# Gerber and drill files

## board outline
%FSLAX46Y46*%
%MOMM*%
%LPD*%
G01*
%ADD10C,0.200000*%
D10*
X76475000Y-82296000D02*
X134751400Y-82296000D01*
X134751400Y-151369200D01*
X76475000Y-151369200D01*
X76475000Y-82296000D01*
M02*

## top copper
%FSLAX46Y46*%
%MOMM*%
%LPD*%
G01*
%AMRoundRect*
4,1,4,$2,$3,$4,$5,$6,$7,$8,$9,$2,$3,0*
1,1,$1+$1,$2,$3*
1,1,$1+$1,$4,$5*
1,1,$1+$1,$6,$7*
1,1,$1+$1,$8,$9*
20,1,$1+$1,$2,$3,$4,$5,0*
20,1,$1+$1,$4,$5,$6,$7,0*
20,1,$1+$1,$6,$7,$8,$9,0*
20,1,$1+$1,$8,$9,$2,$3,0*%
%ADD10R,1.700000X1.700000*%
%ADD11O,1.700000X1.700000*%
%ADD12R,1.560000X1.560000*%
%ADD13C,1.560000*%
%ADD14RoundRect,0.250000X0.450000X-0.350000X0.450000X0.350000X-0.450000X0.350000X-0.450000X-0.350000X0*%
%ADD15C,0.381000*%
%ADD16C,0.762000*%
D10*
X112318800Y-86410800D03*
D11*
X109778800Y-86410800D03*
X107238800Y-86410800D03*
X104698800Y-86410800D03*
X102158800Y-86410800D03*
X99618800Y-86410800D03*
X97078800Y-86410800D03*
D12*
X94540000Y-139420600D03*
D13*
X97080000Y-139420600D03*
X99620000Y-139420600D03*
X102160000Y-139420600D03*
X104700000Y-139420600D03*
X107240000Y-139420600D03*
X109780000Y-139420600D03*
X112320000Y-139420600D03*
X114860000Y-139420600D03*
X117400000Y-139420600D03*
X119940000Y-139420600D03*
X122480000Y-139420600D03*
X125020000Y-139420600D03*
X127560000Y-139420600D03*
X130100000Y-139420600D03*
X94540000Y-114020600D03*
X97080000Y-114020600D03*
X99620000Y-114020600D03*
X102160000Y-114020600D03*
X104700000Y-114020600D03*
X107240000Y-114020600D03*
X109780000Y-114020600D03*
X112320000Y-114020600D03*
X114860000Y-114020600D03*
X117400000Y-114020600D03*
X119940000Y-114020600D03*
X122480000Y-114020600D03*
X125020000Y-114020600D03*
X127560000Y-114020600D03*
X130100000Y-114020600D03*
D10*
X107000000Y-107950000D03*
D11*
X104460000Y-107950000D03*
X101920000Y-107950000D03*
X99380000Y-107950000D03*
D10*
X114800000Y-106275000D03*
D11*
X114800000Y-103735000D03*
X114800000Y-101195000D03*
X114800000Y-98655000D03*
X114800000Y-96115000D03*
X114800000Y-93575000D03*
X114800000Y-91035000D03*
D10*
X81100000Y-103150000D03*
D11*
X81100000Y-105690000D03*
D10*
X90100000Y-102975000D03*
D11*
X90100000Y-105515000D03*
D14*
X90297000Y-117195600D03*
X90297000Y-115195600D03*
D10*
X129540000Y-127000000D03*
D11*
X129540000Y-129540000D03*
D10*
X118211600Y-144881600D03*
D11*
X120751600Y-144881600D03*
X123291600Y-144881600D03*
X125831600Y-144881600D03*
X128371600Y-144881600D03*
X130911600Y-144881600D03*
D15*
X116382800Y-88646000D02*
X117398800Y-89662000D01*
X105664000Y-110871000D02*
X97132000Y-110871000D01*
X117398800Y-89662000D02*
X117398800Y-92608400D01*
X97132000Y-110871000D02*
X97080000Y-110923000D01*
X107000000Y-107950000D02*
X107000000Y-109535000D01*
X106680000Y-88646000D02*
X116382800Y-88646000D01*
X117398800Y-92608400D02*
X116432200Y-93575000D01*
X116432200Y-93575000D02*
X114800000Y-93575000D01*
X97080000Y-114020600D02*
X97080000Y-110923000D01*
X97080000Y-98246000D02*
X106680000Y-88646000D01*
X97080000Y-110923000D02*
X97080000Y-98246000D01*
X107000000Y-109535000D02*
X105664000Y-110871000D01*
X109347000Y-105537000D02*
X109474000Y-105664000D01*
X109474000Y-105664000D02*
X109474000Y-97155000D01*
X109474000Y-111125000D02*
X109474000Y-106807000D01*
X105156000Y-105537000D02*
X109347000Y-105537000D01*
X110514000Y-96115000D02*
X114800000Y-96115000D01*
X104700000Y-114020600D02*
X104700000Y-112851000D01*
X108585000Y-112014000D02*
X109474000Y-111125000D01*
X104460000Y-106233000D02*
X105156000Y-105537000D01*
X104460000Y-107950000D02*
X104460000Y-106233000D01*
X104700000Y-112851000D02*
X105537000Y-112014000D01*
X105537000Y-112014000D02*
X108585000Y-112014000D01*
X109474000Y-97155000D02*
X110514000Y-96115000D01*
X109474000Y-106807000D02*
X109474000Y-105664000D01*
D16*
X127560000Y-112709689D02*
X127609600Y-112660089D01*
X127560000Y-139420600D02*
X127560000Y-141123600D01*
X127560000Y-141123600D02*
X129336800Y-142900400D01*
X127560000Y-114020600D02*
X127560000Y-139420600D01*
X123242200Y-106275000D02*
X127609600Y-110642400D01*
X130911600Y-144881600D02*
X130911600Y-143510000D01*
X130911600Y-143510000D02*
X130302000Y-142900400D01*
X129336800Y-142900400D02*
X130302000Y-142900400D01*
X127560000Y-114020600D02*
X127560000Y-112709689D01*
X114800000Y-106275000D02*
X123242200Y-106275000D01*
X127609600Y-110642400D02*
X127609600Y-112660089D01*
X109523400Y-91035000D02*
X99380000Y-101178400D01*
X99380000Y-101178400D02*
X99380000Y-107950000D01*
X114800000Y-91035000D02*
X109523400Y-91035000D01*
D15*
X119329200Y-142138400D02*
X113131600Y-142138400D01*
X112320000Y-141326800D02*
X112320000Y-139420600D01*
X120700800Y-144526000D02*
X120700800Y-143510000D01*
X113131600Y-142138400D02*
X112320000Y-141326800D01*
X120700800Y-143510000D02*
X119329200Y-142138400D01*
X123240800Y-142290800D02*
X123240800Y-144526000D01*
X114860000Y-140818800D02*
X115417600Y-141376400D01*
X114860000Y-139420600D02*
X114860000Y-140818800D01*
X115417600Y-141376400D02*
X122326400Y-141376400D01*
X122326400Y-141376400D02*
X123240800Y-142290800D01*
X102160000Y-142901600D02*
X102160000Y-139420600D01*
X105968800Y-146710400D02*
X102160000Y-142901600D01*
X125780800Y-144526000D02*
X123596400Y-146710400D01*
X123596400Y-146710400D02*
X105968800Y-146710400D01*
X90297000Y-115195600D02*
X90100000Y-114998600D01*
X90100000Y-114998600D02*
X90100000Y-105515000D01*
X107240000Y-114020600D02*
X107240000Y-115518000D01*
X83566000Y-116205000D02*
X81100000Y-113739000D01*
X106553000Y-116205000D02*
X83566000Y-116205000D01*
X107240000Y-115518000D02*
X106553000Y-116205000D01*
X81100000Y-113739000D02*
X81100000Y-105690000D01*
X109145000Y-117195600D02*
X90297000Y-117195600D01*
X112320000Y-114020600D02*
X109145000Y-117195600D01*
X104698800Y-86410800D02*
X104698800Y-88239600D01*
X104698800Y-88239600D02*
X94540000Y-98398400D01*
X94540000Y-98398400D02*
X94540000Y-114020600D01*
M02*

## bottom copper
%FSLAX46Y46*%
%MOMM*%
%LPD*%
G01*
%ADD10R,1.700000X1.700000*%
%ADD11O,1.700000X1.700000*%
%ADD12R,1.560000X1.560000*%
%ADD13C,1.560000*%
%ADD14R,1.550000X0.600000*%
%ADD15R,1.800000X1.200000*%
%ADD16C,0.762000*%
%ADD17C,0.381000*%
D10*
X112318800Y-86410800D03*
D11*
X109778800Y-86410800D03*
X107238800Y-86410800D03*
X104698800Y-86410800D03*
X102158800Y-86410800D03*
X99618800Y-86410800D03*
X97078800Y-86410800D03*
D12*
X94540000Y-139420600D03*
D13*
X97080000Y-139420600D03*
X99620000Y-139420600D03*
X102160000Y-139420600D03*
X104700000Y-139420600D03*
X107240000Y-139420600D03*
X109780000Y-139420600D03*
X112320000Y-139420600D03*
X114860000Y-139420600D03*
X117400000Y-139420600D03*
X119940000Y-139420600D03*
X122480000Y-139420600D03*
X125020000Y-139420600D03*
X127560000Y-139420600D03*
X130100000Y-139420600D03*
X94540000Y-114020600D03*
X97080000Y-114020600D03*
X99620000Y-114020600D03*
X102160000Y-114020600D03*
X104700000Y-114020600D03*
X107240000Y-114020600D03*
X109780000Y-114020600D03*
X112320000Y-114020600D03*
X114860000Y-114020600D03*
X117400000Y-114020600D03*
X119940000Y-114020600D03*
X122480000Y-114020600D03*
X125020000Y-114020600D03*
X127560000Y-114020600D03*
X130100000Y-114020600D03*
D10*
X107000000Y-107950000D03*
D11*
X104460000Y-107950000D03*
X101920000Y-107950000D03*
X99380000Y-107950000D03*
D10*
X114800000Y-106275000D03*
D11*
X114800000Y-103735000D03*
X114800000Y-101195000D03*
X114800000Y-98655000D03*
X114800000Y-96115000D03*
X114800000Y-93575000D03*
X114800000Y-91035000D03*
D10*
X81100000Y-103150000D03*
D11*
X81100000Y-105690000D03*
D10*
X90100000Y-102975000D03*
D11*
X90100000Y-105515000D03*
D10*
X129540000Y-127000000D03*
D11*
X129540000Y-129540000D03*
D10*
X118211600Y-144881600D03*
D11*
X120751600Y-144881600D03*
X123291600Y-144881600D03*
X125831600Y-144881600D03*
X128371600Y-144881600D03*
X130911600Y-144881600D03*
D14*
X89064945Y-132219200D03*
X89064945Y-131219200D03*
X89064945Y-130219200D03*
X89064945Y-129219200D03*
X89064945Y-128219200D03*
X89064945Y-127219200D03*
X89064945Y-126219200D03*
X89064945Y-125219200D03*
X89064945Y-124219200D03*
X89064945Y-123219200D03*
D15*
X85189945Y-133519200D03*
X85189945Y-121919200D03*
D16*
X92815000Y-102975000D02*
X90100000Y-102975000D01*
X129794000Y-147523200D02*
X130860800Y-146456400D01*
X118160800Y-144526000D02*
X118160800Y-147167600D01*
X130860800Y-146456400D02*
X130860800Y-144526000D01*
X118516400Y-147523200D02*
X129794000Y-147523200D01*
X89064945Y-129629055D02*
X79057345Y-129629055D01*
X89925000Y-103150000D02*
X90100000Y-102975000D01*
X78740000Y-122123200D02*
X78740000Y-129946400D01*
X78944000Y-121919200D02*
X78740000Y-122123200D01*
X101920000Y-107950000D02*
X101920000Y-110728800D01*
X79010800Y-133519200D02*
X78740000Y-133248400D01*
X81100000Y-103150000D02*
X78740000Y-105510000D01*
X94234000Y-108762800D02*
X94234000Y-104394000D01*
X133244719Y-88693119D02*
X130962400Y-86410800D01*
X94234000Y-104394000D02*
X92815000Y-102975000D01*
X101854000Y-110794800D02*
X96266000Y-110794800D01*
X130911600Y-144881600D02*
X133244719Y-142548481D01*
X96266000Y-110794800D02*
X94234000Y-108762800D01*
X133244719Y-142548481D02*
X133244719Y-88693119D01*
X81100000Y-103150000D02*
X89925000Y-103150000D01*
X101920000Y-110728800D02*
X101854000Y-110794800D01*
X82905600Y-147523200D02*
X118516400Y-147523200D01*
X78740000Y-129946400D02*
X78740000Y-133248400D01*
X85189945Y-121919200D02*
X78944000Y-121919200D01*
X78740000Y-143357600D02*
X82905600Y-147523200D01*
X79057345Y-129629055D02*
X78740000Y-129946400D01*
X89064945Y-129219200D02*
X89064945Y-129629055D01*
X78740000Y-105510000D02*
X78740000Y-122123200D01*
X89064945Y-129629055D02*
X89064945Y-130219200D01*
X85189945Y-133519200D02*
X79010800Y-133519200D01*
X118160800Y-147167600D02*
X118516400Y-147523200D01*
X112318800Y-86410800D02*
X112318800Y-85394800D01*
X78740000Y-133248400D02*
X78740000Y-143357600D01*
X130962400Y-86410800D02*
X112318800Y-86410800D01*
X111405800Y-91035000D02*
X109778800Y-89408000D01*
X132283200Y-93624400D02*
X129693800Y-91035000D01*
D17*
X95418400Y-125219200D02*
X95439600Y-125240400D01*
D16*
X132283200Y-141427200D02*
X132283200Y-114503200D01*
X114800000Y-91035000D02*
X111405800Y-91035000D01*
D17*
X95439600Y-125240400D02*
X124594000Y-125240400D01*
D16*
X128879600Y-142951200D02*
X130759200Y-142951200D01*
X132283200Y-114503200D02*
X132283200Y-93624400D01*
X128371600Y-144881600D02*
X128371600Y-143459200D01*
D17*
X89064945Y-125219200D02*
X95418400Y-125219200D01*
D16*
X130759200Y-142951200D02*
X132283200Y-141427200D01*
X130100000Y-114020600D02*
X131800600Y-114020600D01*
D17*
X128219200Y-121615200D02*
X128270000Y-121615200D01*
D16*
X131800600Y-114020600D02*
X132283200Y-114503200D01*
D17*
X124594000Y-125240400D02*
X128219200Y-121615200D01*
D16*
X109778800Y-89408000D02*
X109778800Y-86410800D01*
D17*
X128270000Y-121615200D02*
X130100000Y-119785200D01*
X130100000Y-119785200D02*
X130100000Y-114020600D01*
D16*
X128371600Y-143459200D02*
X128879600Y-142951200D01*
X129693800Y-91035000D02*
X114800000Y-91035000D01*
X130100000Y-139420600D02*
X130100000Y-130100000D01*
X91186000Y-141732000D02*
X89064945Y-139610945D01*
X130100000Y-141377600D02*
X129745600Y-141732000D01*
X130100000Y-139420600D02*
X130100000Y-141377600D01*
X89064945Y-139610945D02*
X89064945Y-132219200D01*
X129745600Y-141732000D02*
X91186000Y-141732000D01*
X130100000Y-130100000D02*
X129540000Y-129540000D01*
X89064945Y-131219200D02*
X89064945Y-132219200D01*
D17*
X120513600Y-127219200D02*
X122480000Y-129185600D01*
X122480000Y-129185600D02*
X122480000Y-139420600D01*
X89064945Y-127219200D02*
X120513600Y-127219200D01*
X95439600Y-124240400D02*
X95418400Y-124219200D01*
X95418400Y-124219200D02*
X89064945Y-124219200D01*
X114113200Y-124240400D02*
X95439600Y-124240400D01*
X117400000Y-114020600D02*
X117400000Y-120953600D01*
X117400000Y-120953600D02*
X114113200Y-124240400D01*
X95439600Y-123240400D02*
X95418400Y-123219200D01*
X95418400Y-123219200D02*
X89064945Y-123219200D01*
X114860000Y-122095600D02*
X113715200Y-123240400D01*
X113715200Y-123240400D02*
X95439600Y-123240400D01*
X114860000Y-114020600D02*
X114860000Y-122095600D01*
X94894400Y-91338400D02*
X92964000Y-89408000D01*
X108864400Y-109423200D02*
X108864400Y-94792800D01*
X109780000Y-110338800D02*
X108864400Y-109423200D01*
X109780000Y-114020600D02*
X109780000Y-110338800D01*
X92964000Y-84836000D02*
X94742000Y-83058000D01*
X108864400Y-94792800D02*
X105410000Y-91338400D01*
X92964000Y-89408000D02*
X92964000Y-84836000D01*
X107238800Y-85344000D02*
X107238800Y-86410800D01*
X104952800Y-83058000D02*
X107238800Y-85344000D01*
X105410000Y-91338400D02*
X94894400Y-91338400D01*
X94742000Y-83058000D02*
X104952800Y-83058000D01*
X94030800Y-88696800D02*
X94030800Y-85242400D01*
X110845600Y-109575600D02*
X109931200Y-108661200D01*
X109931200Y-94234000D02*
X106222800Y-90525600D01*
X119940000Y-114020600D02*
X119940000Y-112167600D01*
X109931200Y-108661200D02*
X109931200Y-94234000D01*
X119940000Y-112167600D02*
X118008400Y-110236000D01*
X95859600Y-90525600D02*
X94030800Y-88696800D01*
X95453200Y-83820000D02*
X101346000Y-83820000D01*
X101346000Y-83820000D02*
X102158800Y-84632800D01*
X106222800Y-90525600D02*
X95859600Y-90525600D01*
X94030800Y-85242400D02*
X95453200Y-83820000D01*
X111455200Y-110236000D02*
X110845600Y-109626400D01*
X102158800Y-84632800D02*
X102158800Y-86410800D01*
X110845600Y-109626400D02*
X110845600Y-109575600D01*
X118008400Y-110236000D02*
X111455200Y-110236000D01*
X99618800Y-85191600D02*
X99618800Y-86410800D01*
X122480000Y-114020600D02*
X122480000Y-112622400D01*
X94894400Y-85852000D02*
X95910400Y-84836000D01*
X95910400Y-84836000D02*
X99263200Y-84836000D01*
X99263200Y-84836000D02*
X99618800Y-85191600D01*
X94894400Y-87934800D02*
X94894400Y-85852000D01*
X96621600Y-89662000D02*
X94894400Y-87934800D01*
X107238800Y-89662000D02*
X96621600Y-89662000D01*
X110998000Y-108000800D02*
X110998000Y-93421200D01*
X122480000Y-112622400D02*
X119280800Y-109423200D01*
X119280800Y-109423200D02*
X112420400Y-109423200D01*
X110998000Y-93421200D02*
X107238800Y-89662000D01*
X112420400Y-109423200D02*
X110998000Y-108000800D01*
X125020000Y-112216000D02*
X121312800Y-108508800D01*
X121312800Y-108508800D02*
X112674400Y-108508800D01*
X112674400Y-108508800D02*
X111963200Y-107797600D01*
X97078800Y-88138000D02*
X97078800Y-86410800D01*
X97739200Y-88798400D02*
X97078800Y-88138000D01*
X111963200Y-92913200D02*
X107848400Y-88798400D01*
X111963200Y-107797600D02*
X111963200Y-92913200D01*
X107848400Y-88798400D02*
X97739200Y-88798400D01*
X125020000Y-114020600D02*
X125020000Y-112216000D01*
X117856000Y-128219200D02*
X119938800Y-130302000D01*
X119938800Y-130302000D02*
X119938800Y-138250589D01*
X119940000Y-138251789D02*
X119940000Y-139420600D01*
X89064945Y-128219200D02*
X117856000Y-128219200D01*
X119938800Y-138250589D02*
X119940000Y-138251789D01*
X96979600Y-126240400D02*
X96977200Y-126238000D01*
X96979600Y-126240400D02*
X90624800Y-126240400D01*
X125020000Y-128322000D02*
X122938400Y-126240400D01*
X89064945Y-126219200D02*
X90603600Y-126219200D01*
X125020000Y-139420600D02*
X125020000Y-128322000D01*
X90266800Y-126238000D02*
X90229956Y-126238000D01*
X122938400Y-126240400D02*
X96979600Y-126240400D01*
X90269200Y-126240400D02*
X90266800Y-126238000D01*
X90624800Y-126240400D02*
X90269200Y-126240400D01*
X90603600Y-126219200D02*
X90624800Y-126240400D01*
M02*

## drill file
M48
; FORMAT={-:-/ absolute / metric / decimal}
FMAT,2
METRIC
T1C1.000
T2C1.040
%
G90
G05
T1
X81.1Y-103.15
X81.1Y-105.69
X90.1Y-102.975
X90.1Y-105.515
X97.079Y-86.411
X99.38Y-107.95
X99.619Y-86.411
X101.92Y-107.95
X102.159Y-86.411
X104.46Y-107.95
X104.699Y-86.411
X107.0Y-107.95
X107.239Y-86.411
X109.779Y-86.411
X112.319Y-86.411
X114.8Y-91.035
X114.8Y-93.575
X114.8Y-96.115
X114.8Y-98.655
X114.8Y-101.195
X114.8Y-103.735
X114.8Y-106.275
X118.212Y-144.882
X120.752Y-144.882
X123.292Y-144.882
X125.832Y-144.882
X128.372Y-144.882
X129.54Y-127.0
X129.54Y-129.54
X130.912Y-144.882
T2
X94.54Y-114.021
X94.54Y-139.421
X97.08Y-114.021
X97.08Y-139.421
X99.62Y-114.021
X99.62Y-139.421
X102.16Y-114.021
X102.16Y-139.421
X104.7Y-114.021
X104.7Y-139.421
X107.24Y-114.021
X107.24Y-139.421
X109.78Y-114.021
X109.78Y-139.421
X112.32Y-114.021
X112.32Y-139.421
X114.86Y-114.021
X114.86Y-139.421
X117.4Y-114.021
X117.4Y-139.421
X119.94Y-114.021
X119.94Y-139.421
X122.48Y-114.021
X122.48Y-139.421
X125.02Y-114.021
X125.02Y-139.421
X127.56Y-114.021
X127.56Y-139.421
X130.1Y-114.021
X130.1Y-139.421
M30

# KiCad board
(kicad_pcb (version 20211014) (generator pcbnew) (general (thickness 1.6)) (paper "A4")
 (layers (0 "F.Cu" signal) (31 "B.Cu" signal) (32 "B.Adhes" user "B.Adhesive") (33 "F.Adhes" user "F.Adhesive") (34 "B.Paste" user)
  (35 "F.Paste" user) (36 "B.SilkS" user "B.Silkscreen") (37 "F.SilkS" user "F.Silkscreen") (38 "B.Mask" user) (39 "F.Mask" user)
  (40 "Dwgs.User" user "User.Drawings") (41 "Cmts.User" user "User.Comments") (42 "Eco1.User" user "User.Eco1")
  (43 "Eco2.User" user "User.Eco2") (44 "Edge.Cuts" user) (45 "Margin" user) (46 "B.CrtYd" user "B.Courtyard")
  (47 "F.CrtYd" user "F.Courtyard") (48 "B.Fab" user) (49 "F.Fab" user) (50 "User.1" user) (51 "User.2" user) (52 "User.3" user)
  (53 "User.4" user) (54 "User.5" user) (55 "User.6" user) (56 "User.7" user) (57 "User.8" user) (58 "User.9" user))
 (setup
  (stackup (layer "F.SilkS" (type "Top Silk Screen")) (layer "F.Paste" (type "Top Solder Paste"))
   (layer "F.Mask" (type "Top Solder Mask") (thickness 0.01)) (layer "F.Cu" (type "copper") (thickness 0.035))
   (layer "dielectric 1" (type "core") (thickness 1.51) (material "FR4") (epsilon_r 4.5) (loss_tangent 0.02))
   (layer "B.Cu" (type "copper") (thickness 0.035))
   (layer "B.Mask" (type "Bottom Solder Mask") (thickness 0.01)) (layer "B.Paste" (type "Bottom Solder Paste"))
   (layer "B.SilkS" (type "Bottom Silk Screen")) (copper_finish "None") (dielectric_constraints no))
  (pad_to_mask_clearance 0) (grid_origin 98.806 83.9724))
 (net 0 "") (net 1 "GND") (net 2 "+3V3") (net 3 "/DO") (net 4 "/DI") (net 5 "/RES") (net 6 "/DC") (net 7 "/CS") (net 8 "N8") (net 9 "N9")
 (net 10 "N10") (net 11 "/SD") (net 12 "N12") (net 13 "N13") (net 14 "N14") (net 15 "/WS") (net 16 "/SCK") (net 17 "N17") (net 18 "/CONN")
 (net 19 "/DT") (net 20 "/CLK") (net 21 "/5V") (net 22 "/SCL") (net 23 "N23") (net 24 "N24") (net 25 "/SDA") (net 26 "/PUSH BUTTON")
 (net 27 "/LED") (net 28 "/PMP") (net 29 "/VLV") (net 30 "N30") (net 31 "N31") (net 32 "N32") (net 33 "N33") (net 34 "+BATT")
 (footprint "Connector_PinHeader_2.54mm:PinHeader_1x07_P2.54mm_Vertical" (layer "F.Cu") (at 112.3188 86.4108 -90)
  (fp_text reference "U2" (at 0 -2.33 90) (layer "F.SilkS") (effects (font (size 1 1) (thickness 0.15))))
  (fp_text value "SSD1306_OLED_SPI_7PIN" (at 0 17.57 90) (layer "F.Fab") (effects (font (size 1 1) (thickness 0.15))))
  (pad "1" thru_hole rect (at 0 0 270) (size 1.7 1.7) (drill 1) (layers *.Cu *.Mask) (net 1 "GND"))
  (pad "2" thru_hole oval (at 0 2.54 270) (size 1.7 1.7) (drill 1) (layers *.Cu *.Mask) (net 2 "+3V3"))
  (pad "3" thru_hole oval (at 0 5.08 270) (size 1.7 1.7) (drill 1) (layers *.Cu *.Mask) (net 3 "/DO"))
  (pad "4" thru_hole oval (at 0 7.62 270) (size 1.7 1.7) (drill 1) (layers *.Cu *.Mask) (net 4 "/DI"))
  (pad "5" thru_hole oval (at 0 10.16 270) (size 1.7 1.7) (drill 1) (layers *.Cu *.Mask) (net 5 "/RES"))
  (pad "6" thru_hole oval (at 0 12.7 270) (size 1.7 1.7) (drill 1) (layers *.Cu *.Mask) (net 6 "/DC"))
  (pad "7" thru_hole oval (at 0 15.24 270) (size 1.7 1.7) (drill 1) (layers *.Cu *.Mask) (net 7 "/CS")))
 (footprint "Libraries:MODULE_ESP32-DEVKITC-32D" (layer "F.Cu") (at 114.3 126.7206 90)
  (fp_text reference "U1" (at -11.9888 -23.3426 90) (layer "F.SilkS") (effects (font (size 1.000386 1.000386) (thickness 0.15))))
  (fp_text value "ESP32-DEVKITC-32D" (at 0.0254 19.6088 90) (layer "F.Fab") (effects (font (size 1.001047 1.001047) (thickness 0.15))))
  (pad "1" thru_hole rect (at -12.7 -19.76 90) (size 1.56 1.56) (drill 1.04) (layers *.Cu *.Mask) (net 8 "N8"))
  (pad "2" thru_hole circle (at -12.7 -17.22 90) (size 1.56 1.56) (drill 1.04) (layers *.Cu *.Mask) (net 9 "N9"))
  (pad "3" thru_hole circle (at -12.7 -14.68 90) (size 1.56 1.56) (drill 1.04) (layers *.Cu *.Mask) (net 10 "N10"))
  (pad "4" thru_hole circle (at -12.7 -12.14 90) (size 1.56 1.56) (drill 1.04) (layers *.Cu *.Mask) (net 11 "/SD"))
  (pad "5" thru_hole circle (at -12.7 -9.6 90) (size 1.56 1.56) (drill 1.04) (layers *.Cu *.Mask) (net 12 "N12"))
  (pad "6" thru_hole circle (at -12.7 -7.06 90) (size 1.56 1.56) (drill 1.04) (layers *.Cu *.Mask) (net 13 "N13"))
  (pad "7" thru_hole circle (at -12.7 -4.52 90) (size 1.56 1.56) (drill 1.04) (layers *.Cu *.Mask) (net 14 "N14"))
  (pad "8" thru_hole circle (at -12.7 -1.98 90) (size 1.56 1.56) (drill 1.04) (layers *.Cu *.Mask) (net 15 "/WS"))
  (pad "9" thru_hole circle (at -12.7 0.56 90) (size 1.56 1.56) (drill 1.04) (layers *.Cu *.Mask) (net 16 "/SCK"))
  (pad "10" thru_hole circle (at -12.7 3.1 90) (size 1.56 1.56) (drill 1.04) (layers *.Cu *.Mask) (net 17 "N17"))
  (pad "11" thru_hole circle (at -12.7 5.64 90) (size 1.56 1.56) (drill 1.04) (layers *.Cu *.Mask) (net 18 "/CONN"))
  (pad "12" thru_hole circle (at -12.7 8.18 90) (size 1.56 1.56) (drill 1.04) (layers *.Cu *.Mask) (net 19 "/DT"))
  (pad "13" thru_hole circle (at -12.7 10.72 90) (size 1.56 1.56) (drill 1.04) (layers *.Cu *.Mask) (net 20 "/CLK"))
  (pad "14" thru_hole circle (at -12.7 13.26 90) (size 1.56 1.56) (drill 1.04) (layers *.Cu *.Mask) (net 1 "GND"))
  (pad "15" thru_hole circle (at -12.7 15.8 90) (size 1.56 1.56) (drill 1.04) (layers *.Cu *.Mask) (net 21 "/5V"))
  (pad "16" thru_hole circle (at 12.7 -19.76 90) (size 1.56 1.56) (drill 1.04) (layers *.Cu *.Mask) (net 4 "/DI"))
  (pad "17" thru_hole circle (at 12.7 -17.22 90) (size 1.56 1.56) (drill 1.04) (layers *.Cu *.Mask) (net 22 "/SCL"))
  (pad "18" thru_hole circle (at 12.7 -14.68 90) (size 1.56 1.56) (drill 1.04) (layers *.Cu *.Mask) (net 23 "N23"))
  (pad "19" thru_hole circle (at 12.7 -12.14 90) (size 1.56 1.56) (drill 1.04) (layers *.Cu *.Mask) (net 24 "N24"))
  (pad "20" thru_hole circle (at 12.7 -9.6 90) (size 1.56 1.56) (drill 1.04) (layers *.Cu *.Mask) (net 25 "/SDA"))
  (pad "21" thru_hole circle (at 12.7 -7.06 90) (size 1.56 1.56) (drill 1.04) (layers *.Cu *.Mask) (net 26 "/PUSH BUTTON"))
  (pad "22" thru_hole circle (at 12.7 -4.52 90) (size 1.56 1.56) (drill 1.04) (layers *.Cu *.Mask) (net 3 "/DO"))
  (pad "23" thru_hole circle (at 12.7 -1.98 90) (size 1.56 1.56) (drill 1.04) (layers *.Cu *.Mask) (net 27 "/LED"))
  (pad "24" thru_hole circle (at 12.7 0.56 90) (size 1.56 1.56) (drill 1.04) (layers *.Cu *.Mask) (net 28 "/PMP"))
  (pad "25" thru_hole circle (at 12.7 3.1 90) (size 1.56 1.56) (drill 1.04) (layers *.Cu *.Mask) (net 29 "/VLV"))
  (pad "26" thru_hole circle (at 12.7 5.64 90) (size 1.56 1.56) (drill 1.04) (layers *.Cu *.Mask) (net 5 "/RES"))
  (pad "27" thru_hole circle (at 12.7 8.18 90) (size 1.56 1.56) (drill 1.04) (layers *.Cu *.Mask) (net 6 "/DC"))
  (pad "28" thru_hole circle (at 12.7 10.72 90) (size 1.56 1.56) (drill 1.04) (layers *.Cu *.Mask) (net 7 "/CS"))
  (pad "29" thru_hole circle (at 12.7 13.26 90) (size 1.56 1.56) (drill 1.04) (layers *.Cu *.Mask) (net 1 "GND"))
  (pad "30" thru_hole circle (at 12.7 15.8 90) (size 1.56 1.56) (drill 1.04) (layers *.Cu *.Mask) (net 2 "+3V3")))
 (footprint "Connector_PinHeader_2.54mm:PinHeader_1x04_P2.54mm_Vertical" (layer "F.Cu") (at 107 107.95 -90)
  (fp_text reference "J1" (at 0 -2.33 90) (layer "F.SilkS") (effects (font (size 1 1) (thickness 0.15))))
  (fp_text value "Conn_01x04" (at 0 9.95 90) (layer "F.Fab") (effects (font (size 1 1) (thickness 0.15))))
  (pad "1" thru_hole rect (at 0 0 270) (size 1.7 1.7) (drill 1) (layers *.Cu *.Mask) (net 22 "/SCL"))
  (pad "2" thru_hole oval (at 0 2.54 270) (size 1.7 1.7) (drill 1) (layers *.Cu *.Mask) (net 25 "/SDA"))
  (pad "3" thru_hole oval (at 0 5.08 270) (size 1.7 1.7) (drill 1) (layers *.Cu *.Mask) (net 1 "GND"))
  (pad "4" thru_hole oval (at 0 7.62 270) (size 1.7 1.7) (drill 1) (layers *.Cu *.Mask) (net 2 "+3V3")))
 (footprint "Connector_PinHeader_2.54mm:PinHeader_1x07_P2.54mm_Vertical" (layer "F.Cu") (at 114.8 106.275 180)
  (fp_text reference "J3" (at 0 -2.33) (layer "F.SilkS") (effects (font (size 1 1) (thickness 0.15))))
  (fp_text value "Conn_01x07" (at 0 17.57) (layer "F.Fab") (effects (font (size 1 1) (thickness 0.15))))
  (pad "1" thru_hole rect (at 0 0 180) (size 1.7 1.7) (drill 1) (layers *.Cu *.Mask) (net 1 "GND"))
  (pad "2" thru_hole oval (at 0 2.54 180) (size 1.7 1.7) (drill 1) (layers *.Cu *.Mask) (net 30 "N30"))
  (pad "3" thru_hole oval (at 0 5.08 180) (size 1.7 1.7) (drill 1) (layers *.Cu *.Mask) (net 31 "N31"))
  (pad "4" thru_hole oval (at 0 7.62 180) (size 1.7 1.7) (drill 1) (layers *.Cu *.Mask) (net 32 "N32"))
  (pad "5" thru_hole oval (at 0 10.16 180) (size 1.7 1.7) (drill 1) (layers *.Cu *.Mask) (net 25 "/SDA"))
  (pad "6" thru_hole oval (at 0 12.7 180) (size 1.7 1.7) (drill 1) (layers *.Cu *.Mask) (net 22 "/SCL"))
  (pad "7" thru_hole oval (at 0 15.24 180) (size 1.7 1.7) (drill 1) (layers *.Cu *.Mask) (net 2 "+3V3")))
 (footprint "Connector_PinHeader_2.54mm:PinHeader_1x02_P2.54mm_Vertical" (layer "F.Cu") (at 81.1 103.15)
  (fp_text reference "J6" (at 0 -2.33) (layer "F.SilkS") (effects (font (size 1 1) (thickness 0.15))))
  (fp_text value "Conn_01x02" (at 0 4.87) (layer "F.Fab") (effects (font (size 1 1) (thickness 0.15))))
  (pad "1" thru_hole rect (at 0 0) (size 1.7 1.7) (drill 1) (layers *.Cu *.Mask) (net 1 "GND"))
  (pad "2" thru_hole oval (at 0 2.54) (size 1.7 1.7) (drill 1) (layers *.Cu *.Mask) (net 26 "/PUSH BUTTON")))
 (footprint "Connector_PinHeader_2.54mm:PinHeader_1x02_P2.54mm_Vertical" (layer "F.Cu") (at 90.1 102.975)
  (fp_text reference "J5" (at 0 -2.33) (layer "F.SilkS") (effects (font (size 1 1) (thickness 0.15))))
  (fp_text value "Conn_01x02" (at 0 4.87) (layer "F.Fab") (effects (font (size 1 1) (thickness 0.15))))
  (pad "1" thru_hole rect (at 0 0) (size 1.7 1.7) (drill 1) (layers *.Cu *.Mask) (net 1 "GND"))
  (pad "2" thru_hole oval (at 0 2.54) (size 1.7 1.7) (drill 1) (layers *.Cu *.Mask) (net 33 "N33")))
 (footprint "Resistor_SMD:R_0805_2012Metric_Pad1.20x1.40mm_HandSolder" (layer "F.Cu") (at 90.297 116.1956 90)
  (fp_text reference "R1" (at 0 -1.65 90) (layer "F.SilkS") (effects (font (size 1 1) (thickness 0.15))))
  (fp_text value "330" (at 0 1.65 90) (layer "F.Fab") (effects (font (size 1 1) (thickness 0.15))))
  (pad "1" smd roundrect (at -1 0 90) (size 1.2 1.4) (layers "F.Cu" "F.Paste" "F.Mask") (roundrect_rratio 0.208333) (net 27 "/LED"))
  (pad "2" smd roundrect (at 1 0 90) (size 1.2 1.4) (layers "F.Cu" "F.Paste" "F.Mask") (roundrect_rratio 0.208333) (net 33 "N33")))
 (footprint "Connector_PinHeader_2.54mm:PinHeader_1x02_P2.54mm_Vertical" (layer "F.Cu") (at 129.54 127)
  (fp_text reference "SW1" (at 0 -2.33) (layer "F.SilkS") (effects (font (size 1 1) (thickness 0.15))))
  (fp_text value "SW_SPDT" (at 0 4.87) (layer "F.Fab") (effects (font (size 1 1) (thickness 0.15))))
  (pad "1" thru_hole rect (at 0 0) (size 1.7 1.7) (drill 1) (layers *.Cu *.Mask) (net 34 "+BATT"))
  (pad "3" thru_hole oval (at 0 2.54) (size 1.7 1.7) (drill 1) (layers *.Cu *.Mask) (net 21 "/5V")))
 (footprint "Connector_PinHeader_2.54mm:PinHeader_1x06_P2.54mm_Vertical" (layer "B.Cu") (at 118.2116 144.8816 -90)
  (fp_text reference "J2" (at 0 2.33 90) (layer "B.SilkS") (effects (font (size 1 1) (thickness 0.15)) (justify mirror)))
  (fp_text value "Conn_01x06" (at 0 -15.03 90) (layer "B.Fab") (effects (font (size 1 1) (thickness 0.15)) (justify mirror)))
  (pad "1" thru_hole rect (at 0 0 270) (size 1.7 1.7) (drill 1) (layers *.Cu *.Mask) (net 1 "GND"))
  (pad "2" thru_hole oval (at 0 -2.54 270) (size 1.7 1.7) (drill 1) (layers *.Cu *.Mask) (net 15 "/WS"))
  (pad "3" thru_hole oval (at 0 -5.08 270) (size 1.7 1.7) (drill 1) (layers *.Cu *.Mask) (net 16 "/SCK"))
  (pad "4" thru_hole oval (at 0 -7.62 270) (size 1.7 1.7) (drill 1) (layers *.Cu *.Mask) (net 11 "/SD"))
  (pad "5" thru_hole oval (at 0 -10.16 270) (size 1.7 1.7) (drill 1) (layers *.Cu *.Mask) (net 2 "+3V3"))
  (pad "6" thru_hole oval (at 0 -12.7 270) (size 1.7 1.7) (drill 1) (layers *.Cu *.Mask) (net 1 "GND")))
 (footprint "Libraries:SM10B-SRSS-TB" (layer "B.Cu") (at 88.722945 133.7192 90)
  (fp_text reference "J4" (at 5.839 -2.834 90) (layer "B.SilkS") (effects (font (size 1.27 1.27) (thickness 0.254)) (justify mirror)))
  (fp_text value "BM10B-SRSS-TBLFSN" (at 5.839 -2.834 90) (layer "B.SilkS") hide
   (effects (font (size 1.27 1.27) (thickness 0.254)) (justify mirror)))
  (pad "1" smd rect locked (at 1.5 0.342 90) (size 0.6 1.55) (layers "B.Cu" "B.Paste" "B.Mask") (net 21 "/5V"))
  (pad "2" smd rect locked (at 2.5 0.342 90) (size 0.6 1.55) (layers "B.Cu" "B.Paste" "B.Mask") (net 21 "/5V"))
  (pad "3" smd rect locked (at 3.5 0.342 90) (size 0.6 1.55) (layers "B.Cu" "B.Paste" "B.Mask") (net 1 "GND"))
  (pad "4" smd rect locked (at 4.5 0.342 90) (size 0.6 1.55) (layers "B.Cu" "B.Paste" "B.Mask") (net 1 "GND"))
  (pad "5" smd rect locked (at 5.5 0.342 90) (size 0.6 1.55) (layers "B.Cu" "B.Paste" "B.Mask") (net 18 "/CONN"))
  (pad "6" smd rect locked (at 6.5 0.342 90) (size 0.6 1.55) (layers "B.Cu" "B.Paste" "B.Mask") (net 19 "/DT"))
  (pad "7" smd rect locked (at 7.5 0.342 90) (size 0.6 1.55) (layers "B.Cu" "B.Paste" "B.Mask") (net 20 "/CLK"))
  (pad "8" smd rect locked (at 8.5 0.342 90) (size 0.6 1.55) (layers "B.Cu" "B.Paste" "B.Mask") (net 2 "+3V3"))
  (pad "9" smd rect locked (at 9.5 0.342 90) (size 0.6 1.55) (layers "B.Cu" "B.Paste" "B.Mask") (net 29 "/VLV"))
  (pad "10" smd rect locked (at 10.5 0.342 90) (size 0.6 1.55) (layers "B.Cu" "B.Paste" "B.Mask") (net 28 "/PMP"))
  (pad "11" smd rect locked (at 0.2 -3.533 90) (size 1.2 1.8) (layers "B.Cu" "B.Paste" "B.Mask"))
  (pad "12" smd rect locked (at 11.8 -3.533 90) (size 1.2 1.8) (layers "B.Cu" "B.Paste" "B.Mask")))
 (gr_rect (start 76.475 82.296) (end 134.7514 151.3692) (layer "Edge.Cuts") (width 0.2) (fill none))
 (segment (start 116.3828 88.646) (end 117.3988 89.662) (width 0.381) (layer "F.Cu") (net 22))
 (segment (start 105.664 110.871) (end 97.132 110.871) (width 0.381) (layer "F.Cu") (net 22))
 (segment (start 117.3988 89.662) (end 117.3988 92.6084) (width 0.381) (layer "F.Cu") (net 22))
 (segment (start 97.132 110.871) (end 97.08 110.923) (width 0.381) (layer "F.Cu") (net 22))
 (segment (start 107 107.95) (end 107 109.535) (width 0.381) (layer "F.Cu") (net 22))
 (segment (start 106.68 88.646) (end 116.3828 88.646) (width 0.381) (layer "F.Cu") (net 22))
 (segment (start 117.3988 92.6084) (end 116.4322 93.575) (width 0.381) (layer "F.Cu") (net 22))
 (segment (start 116.4322 93.575) (end 114.8 93.575) (width 0.381) (layer "F.Cu") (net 22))
 (segment (start 97.08 114.0206) (end 97.08 110.923) (width 0.381) (layer "F.Cu") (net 22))
 (segment (start 97.08 98.246) (end 106.68 88.646) (width 0.381) (layer "F.Cu") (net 22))
 (segment (start 97.08 110.923) (end 97.08 98.246) (width 0.381) (layer "F.Cu") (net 22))
 (segment (start 107 109.535) (end 105.664 110.871) (width 0.381) (layer "F.Cu") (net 22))
 (segment (start 109.347 105.537) (end 109.474 105.664) (width 0.381) (layer "F.Cu") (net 25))
 (segment (start 109.474 105.664) (end 109.474 97.155) (width 0.381) (layer "F.Cu") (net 25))
 (segment (start 109.474 111.125) (end 109.474 106.807) (width 0.381) (layer "F.Cu") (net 25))
 (segment (start 105.156 105.537) (end 109.347 105.537) (width 0.381) (layer "F.Cu") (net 25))
 (segment (start 110.514 96.115) (end 114.8 96.115) (width 0.381) (layer "F.Cu") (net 25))
 (segment (start 104.7 114.0206) (end 104.7 112.851) (width 0.381) (layer "F.Cu") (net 25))
 (segment (start 108.585 112.014) (end 109.474 111.125) (width 0.381) (layer "F.Cu") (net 25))
 (segment (start 104.46 106.233) (end 105.156 105.537) (width 0.381) (layer "F.Cu") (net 25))
 (segment (start 104.46 107.95) (end 104.46 106.233) (width 0.381) (layer "F.Cu") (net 25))
 (segment (start 104.7 112.851) (end 105.537 112.014) (width 0.381) (layer "F.Cu") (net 25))
 (segment (start 105.537 112.014) (end 108.585 112.014) (width 0.381) (layer "F.Cu") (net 25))
 (segment (start 109.474 97.155) (end 110.514 96.115) (width 0.381) (layer "F.Cu") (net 25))
 (segment (start 109.474 106.807) (end 109.474 105.664) (width 0.381) (layer "F.Cu") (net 25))
 (segment (start 127.56 112.709689) (end 127.6096 112.660089) (width 0.762) (layer "F.Cu") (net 1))
 (segment (start 127.56 139.4206) (end 127.56 141.1236) (width 0.762) (layer "F.Cu") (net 1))
 (segment (start 127.56 141.1236) (end 129.3368 142.9004) (width 0.762) (layer "F.Cu") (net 1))
 (segment (start 127.56 114.0206) (end 127.56 139.4206) (width 0.762) (layer "F.Cu") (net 1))
 (segment (start 123.2422 106.275) (end 127.6096 110.6424) (width 0.762) (layer "F.Cu") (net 1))
 (segment (start 130.9116 144.8816) (end 130.9116 143.51) (width 0.762) (layer "F.Cu") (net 1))
 (segment (start 130.9116 143.51) (end 130.302 142.9004) (width 0.762) (layer "F.Cu") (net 1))
 (segment (start 129.3368 142.9004) (end 130.302 142.9004) (width 0.762) (layer "F.Cu") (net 1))
 (segment (start 127.56 114.0206) (end 127.56 112.709689) (width 0.762) (layer "F.Cu") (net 1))
 (segment (start 114.8 106.275) (end 123.2422 106.275) (width 0.762) (layer "F.Cu") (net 1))
 (segment (start 127.6096 110.6424) (end 127.6096 112.660089) (width 0.762) (layer "F.Cu") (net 1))
 (segment (start 92.815 102.975) (end 90.1 102.975) (width 0.762) (layer "B.Cu") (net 1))
 (segment (start 129.794 147.5232) (end 130.8608 146.4564) (width 0.762) (layer "B.Cu") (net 1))
 (segment (start 118.1608 144.526) (end 118.1608 147.1676) (width 0.762) (layer "B.Cu") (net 1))
 (segment (start 130.8608 146.4564) (end 130.8608 144.526) (width 0.762) (layer "B.Cu") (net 1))
 (segment (start 118.5164 147.5232) (end 129.794 147.5232) (width 0.762) (layer "B.Cu") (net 1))
 (segment (start 89.064945 129.629055) (end 79.057345 129.629055) (width 0.762) (layer "B.Cu") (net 1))
 (segment (start 89.925 103.15) (end 90.1 102.975) (width 0.762) (layer "B.Cu") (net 1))
 (segment (start 78.74 122.1232) (end 78.74 129.9464) (width 0.762) (layer "B.Cu") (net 1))
 (segment (start 78.944 121.9192) (end 78.74 122.1232) (width 0.762) (layer "B.Cu") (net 1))
 (segment (start 101.92 107.95) (end 101.92 110.7288) (width 0.762) (layer "B.Cu") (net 1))
 (segment (start 79.0108 133.5192) (end 78.74 133.2484) (width 0.762) (layer "B.Cu") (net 1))
 (segment (start 81.1 103.15) (end 78.74 105.51) (width 0.762) (layer "B.Cu") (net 1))
 (segment (start 94.234 108.7628) (end 94.234 104.394) (width 0.762) (layer "B.Cu") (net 1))
 (segment (start 133.244719 88.693119) (end 130.9624 86.4108) (width 0.762) (layer "B.Cu") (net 1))
 (segment (start 94.234 104.394) (end 92.815 102.975) (width 0.762) (layer "B.Cu") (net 1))
 (segment (start 101.854 110.7948) (end 96.266 110.7948) (width 0.762) (layer "B.Cu") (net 1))
 (segment (start 130.9116 144.8816) (end 133.244719 142.548481) (width 0.762) (layer "B.Cu") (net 1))
 (segment (start 96.266 110.7948) (end 94.234 108.7628) (width 0.762) (layer "B.Cu") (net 1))
 (segment (start 133.244719 142.548481) (end 133.244719 88.693119) (width 0.762) (layer "B.Cu") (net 1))
 (segment (start 81.1 103.15) (end 89.925 103.15) (width 0.762) (layer "B.Cu") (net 1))
 (segment (start 101.92 110.7288) (end 101.854 110.7948) (width 0.762) (layer "B.Cu") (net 1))
 (segment (start 82.9056 147.5232) (end 118.5164 147.5232) (width 0.762) (layer "B.Cu") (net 1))
 (segment (start 78.74 129.9464) (end 78.74 133.2484) (width 0.762) (layer "B.Cu") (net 1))
 (segment (start 85.189945 121.9192) (end 78.944 121.9192) (width 0.762) (layer "B.Cu") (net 1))
 (segment (start 78.74 143.3576) (end 82.9056 147.5232) (width 0.762) (layer "B.Cu") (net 1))
 (segment (start 79.057345 129.629055) (end 78.74 129.9464) (width 0.762) (layer "B.Cu") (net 1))
 (segment (start 89.064945 129.2192) (end 89.064945 129.629055) (width 0.762) (layer "B.Cu") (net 1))
 (segment (start 78.74 105.51) (end 78.74 122.1232) (width 0.762) (layer "B.Cu") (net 1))
 (segment (start 89.064945 129.629055) (end 89.064945 130.2192) (width 0.762) (layer "B.Cu") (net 1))
 (segment (start 85.189945 133.5192) (end 79.0108 133.5192) (width 0.762) (layer "B.Cu") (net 1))
 (segment (start 118.1608 147.1676) (end 118.5164 147.5232) (width 0.762) (layer "B.Cu") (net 1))
 (segment (start 112.3188 86.4108) (end 112.3188 85.3948) (width 0.762) (layer "B.Cu") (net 1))
 (segment (start 78.74 133.2484) (end 78.74 143.3576) (width 0.762) (layer "B.Cu") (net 1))
 (segment (start 130.9624 86.4108) (end 112.3188 86.4108) (width 0.762) (layer "B.Cu") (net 1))
 (segment (start 109.5234 91.035) (end 99.38 101.1784) (width 0.762) (layer "F.Cu") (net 2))
 (segment (start 99.38 101.1784) (end 99.38 107.95) (width 0.762) (layer "F.Cu") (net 2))
 (segment (start 114.8 91.035) (end 109.5234 91.035) (width 0.762) (layer "F.Cu") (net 2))
 (segment (start 111.4058 91.035) (end 109.7788 89.408) (width 0.762) (layer "B.Cu") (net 2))
 (segment (start 132.2832 93.6244) (end 129.6938 91.035) (width 0.762) (layer "B.Cu") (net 2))
 (segment (start 95.4184 125.2192) (end 95.4396 125.2404) (width 0.381) (layer "B.Cu") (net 2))
 (segment (start 132.2832 141.4272) (end 132.2832 114.5032) (width 0.762) (layer "B.Cu") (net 2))
 (segment (start 114.8 91.035) (end 111.4058 91.035) (width 0.762) (layer "B.Cu") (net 2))
 (segment (start 95.4396 125.2404) (end 124.594 125.2404) (width 0.381) (layer "B.Cu") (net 2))
 (segment (start 128.8796 142.9512) (end 130.7592 142.9512) (width 0.762) (layer "B.Cu") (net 2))
 (segment (start 132.2832 114.5032) (end 132.2832 93.6244) (width 0.762) (layer "B.Cu") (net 2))
 (segment (start 128.3716 144.8816) (end 128.3716 143.4592) (width 0.762) (layer "B.Cu") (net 2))
 (segment (start 89.064945 125.2192) (end 95.4184 125.2192) (width 0.381) (layer "B.Cu") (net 2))
 (segment (start 130.7592 142.9512) (end 132.2832 141.4272) (width 0.762) (layer "B.Cu") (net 2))
 (segment (start 130.1 114.0206) (end 131.8006 114.0206) (width 0.762) (layer "B.Cu") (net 2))
 (segment (start 128.2192 121.6152) (end 128.27 121.6152) (width 0.381) (layer "B.Cu") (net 2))
 (segment (start 131.8006 114.0206) (end 132.2832 114.5032) (width 0.762) (layer "B.Cu") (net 2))
 (segment (start 124.594 125.2404) (end 128.2192 121.6152) (width 0.381) (layer "B.Cu") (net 2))
 (segment (start 109.7788 89.408) (end 109.7788 86.4108) (width 0.762) (layer "B.Cu") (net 2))
 (segment (start 128.27 121.6152) (end 130.1 119.7852) (width 0.381) (layer "B.Cu") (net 2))
 (segment (start 130.1 119.7852) (end 130.1 114.0206) (width 0.381) (layer "B.Cu") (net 2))
 (segment (start 128.3716 143.4592) (end 128.8796 142.9512) (width 0.762) (layer "B.Cu") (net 2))
 (segment (start 129.6938 91.035) (end 114.8 91.035) (width 0.762) (layer "B.Cu") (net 2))
 (segment (start 119.3292 142.1384) (end 113.1316 142.1384) (width 0.381) (layer "F.Cu") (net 15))
 (segment (start 112.32 141.3268) (end 112.32 139.4206) (width 0.381) (layer "F.Cu") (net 15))
 (segment (start 120.7008 144.526) (end 120.7008 143.51) (width 0.381) (layer "F.Cu") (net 15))
 (segment (start 113.1316 142.1384) (end 112.32 141.3268) (width 0.381) (layer "F.Cu") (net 15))
 (segment (start 120.7008 143.51) (end 119.3292 142.1384) (width 0.381) (layer "F.Cu") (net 15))
 (segment (start 123.2408 142.2908) (end 123.2408 144.526) (width 0.381) (layer "F.Cu") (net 16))
 (segment (start 114.86 140.8188) (end 115.4176 141.3764) (width 0.381) (layer "F.Cu") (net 16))
 (segment (start 114.86 139.4206) (end 114.86 140.8188) (width 0.381) (layer "F.Cu") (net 16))
 (segment (start 115.4176 141.3764) (end 122.3264 141.3764) (width 0.381) (layer "F.Cu") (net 16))
 (segment (start 122.3264 141.3764) (end 123.2408 142.2908) (width 0.381) (layer "F.Cu") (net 16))
 (segment (start 102.16 142.9016) (end 102.16 139.4206) (width 0.381) (layer "F.Cu") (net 11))
 (segment (start 105.9688 146.7104) (end 102.16 142.9016) (width 0.381) (layer "F.Cu") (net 11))
 (segment (start 125.7808 144.526) (end 123.5964 146.7104) (width 0.381) (layer "F.Cu") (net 11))
 (segment (start 123.5964 146.7104) (end 105.9688 146.7104) (width 0.381) (layer "F.Cu") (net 11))
 (segment (start 130.1 139.4206) (end 130.1 130.1) (width 0.762) (layer "B.Cu") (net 21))
 (segment (start 91.186 141.732) (end 89.064945 139.610945) (width 0.762) (layer "B.Cu") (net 21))
 (segment (start 130.1 141.3776) (end 129.7456 141.732) (width 0.762) (layer "B.Cu") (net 21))
 (segment (start 130.1 139.4206) (end 130.1 141.3776) (width 0.762) (layer "B.Cu") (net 21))
 (segment (start 89.064945 139.610945) (end 89.064945 132.2192) (width 0.762) (layer "B.Cu") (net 21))
 (segment (start 129.7456 141.732) (end 91.186 141.732) (width 0.762) (layer "B.Cu") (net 21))
 (segment (start 130.1 130.1) (end 129.54 129.54) (width 0.762) (layer "B.Cu") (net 21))
 (segment (start 89.064945 131.2192) (end 89.064945 132.2192) (width 0.762) (layer "B.Cu") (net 21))
 (segment (start 120.5136 127.2192) (end 122.48 129.1856) (width 0.381) (layer "B.Cu") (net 19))
 (segment (start 122.48 129.1856) (end 122.48 139.4206) (width 0.381) (layer "B.Cu") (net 19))
 (segment (start 89.064945 127.2192) (end 120.5136 127.2192) (width 0.381) (layer "B.Cu") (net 19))
 (segment (start 95.4396 124.2404) (end 95.4184 124.2192) (width 0.381) (layer "B.Cu") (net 29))
 (segment (start 95.4184 124.2192) (end 89.064945 124.2192) (width 0.381) (layer "B.Cu") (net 29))
 (segment (start 114.1132 124.2404) (end 95.4396 124.2404) (width 0.381) (layer "B.Cu") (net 29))
 (segment (start 117.4 114.0206) (end 117.4 120.9536) (width 0.381) (layer "B.Cu") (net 29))
 (segment (start 117.4 120.9536) (end 114.1132 124.2404) (width 0.381) (layer "B.Cu") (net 29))
 (segment (start 95.4396 123.2404) (end 95.4184 123.2192) (width 0.381) (layer "B.Cu") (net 28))
 (segment (start 95.4184 123.2192) (end 89.064945 123.2192) (width 0.381) (layer "B.Cu") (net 28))
 (segment (start 114.86 122.0956) (end 113.7152 123.2404) (width 0.381) (layer "B.Cu") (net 28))
 (segment (start 113.7152 123.2404) (end 95.4396 123.2404) (width 0.381) (layer "B.Cu") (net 28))
 (segment (start 114.86 114.0206) (end 114.86 122.0956) (width 0.381) (layer "B.Cu") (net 28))
 (segment (start 90.297 115.1956) (end 90.1 114.9986) (width 0.381) (layer "F.Cu") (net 33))
 (segment (start 90.1 114.9986) (end 90.1 105.515) (width 0.381) (layer "F.Cu") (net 33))
 (segment (start 107.24 114.0206) (end 107.24 115.518) (width 0.381) (layer "F.Cu") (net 26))
 (segment (start 83.566 116.205) (end 81.1 113.739) (width 0.381) (layer "F.Cu") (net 26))
 (segment (start 106.553 116.205) (end 83.566 116.205) (width 0.381) (layer "F.Cu") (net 26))
 (segment (start 107.24 115.518) (end 106.553 116.205) (width 0.381) (layer "F.Cu") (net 26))
 (segment (start 81.1 113.739) (end 81.1 105.69) (width 0.381) (layer "F.Cu") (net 26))
 (segment (start 109.145 117.1956) (end 90.297 117.1956) (width 0.381) (layer "F.Cu") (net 27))
 (segment (start 112.32 114.0206) (end 109.145 117.1956) (width 0.381) (layer "F.Cu") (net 27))
 (segment (start 104.6988 86.4108) (end 104.6988 88.2396) (width 0.381) (layer "F.Cu") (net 4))
 (segment (start 104.6988 88.2396) (end 94.54 98.3984) (width 0.381) (layer "F.Cu") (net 4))
 (segment (start 94.54 98.3984) (end 94.54 114.0206) (width 0.381) (layer "F.Cu") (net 4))
 (segment (start 94.8944 91.3384) (end 92.964 89.408) (width 0.381) (layer "B.Cu") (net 3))
 (segment (start 108.8644 109.4232) (end 108.8644 94.7928) (width 0.381) (layer "B.Cu") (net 3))
 (segment (start 109.78 110.3388) (end 108.8644 109.4232) (width 0.381) (layer "B.Cu") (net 3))
 (segment (start 109.78 114.0206) (end 109.78 110.3388) (width 0.381) (layer "B.Cu") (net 3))
 (segment (start 92.964 84.836) (end 94.742 83.058) (width 0.381) (layer "B.Cu") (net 3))
 (segment (start 108.8644 94.7928) (end 105.41 91.3384) (width 0.381) (layer "B.Cu") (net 3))
 (segment (start 92.964 89.408) (end 92.964 84.836) (width 0.381) (layer "B.Cu") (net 3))
 (segment (start 107.2388 85.344) (end 107.2388 86.4108) (width 0.381) (layer "B.Cu") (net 3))
 (segment (start 104.9528 83.058) (end 107.2388 85.344) (width 0.381) (layer "B.Cu") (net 3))
 (segment (start 105.41 91.3384) (end 94.8944 91.3384) (width 0.381) (layer "B.Cu") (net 3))
 (segment (start 94.742 83.058) (end 104.9528 83.058) (width 0.381) (layer "B.Cu") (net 3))
 (segment (start 94.0308 88.6968) (end 94.0308 85.2424) (width 0.381) (layer "B.Cu") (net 5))
 (segment (start 110.8456 109.5756) (end 109.9312 108.6612) (width 0.381) (layer "B.Cu") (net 5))
 (segment (start 109.9312 94.234) (end 106.2228 90.5256) (width 0.381) (layer "B.Cu") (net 5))
 (segment (start 119.94 114.0206) (end 119.94 112.1676) (width 0.381) (layer "B.Cu") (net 5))
 (segment (start 109.9312 108.6612) (end 109.9312 94.234) (width 0.381) (layer "B.Cu") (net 5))
 (segment (start 119.94 112.1676) (end 118.0084 110.236) (width 0.381) (layer "B.Cu") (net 5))
 (segment (start 95.8596 90.5256) (end 94.0308 88.6968) (width 0.381) (layer "B.Cu") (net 5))
 (segment (start 95.4532 83.82) (end 101.346 83.82) (width 0.381) (layer "B.Cu") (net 5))
 (segment (start 101.346 83.82) (end 102.1588 84.6328) (width 0.381) (layer "B.Cu") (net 5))
 (segment (start 106.2228 90.5256) (end 95.8596 90.5256) (width 0.381) (layer "B.Cu") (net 5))
 (segment (start 94.0308 85.2424) (end 95.4532 83.82) (width 0.381) (layer "B.Cu") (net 5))
 (segment (start 111.4552 110.236) (end 110.8456 109.6264) (width 0.381) (layer "B.Cu") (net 5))
 (segment (start 102.1588 84.6328) (end 102.1588 86.4108) (width 0.381) (layer "B.Cu") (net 5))
 (segment (start 110.8456 109.6264) (end 110.8456 109.5756) (width 0.381) (layer "B.Cu") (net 5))
 (segment (start 118.0084 110.236) (end 111.4552 110.236) (width 0.381) (layer "B.Cu") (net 5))
 (segment (start 99.6188 85.1916) (end 99.6188 86.4108) (width 0.381) (layer "B.Cu") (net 6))
 (segment (start 122.48 114.0206) (end 122.48 112.6224) (width 0.381) (layer "B.Cu") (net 6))
 (segment (start 94.8944 85.852) (end 95.9104 84.836) (width 0.381) (layer "B.Cu") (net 6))
 (segment (start 95.9104 84.836) (end 99.2632 84.836) (width 0.381) (layer "B.Cu") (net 6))
 (segment (start 99.2632 84.836) (end 99.6188 85.1916) (width 0.381) (layer "B.Cu") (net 6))
 (segment (start 94.8944 87.9348) (end 94.8944 85.852) (width 0.381) (layer "B.Cu") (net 6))
 (segment (start 96.6216 89.662) (end 94.8944 87.9348) (width 0.381) (layer "B.Cu") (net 6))
 (segment (start 107.2388 89.662) (end 96.6216 89.662) (width 0.381) (layer "B.Cu") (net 6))
 (segment (start 110.998 108.0008) (end 110.998 93.4212) (width 0.381) (layer "B.Cu") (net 6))
 (segment (start 122.48 112.6224) (end 119.2808 109.4232) (width 0.381) (layer "B.Cu") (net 6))
 (segment (start 119.2808 109.4232) (end 112.4204 109.4232) (width 0.381) (layer "B.Cu") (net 6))
 (segment (start 110.998 93.4212) (end 107.2388 89.662) (width 0.381) (layer "B.Cu") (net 6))
 (segment (start 112.4204 109.4232) (end 110.998 108.0008) (width 0.381) (layer "B.Cu") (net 6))
 (segment (start 125.02 112.216) (end 121.3128 108.5088) (width 0.381) (layer "B.Cu") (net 7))
 (segment (start 121.3128 108.5088) (end 112.6744 108.5088) (width 0.381) (layer "B.Cu") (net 7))
 (segment (start 112.6744 108.5088) (end 111.9632 107.7976) (width 0.381) (layer "B.Cu") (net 7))
 (segment (start 97.0788 88.138) (end 97.0788 86.4108) (width 0.381) (layer "B.Cu") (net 7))
 (segment (start 97.7392 88.7984) (end 97.0788 88.138) (width 0.381) (layer "B.Cu") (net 7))
 (segment (start 111.9632 92.9132) (end 107.8484 88.7984) (width 0.381) (layer "B.Cu") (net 7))
 (segment (start 111.9632 107.7976) (end 111.9632 92.9132) (width 0.381) (layer "B.Cu") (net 7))
 (segment (start 107.8484 88.7984) (end 97.7392 88.7984) (width 0.381) (layer "B.Cu") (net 7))
 (segment (start 125.02 114.0206) (end 125.02 112.216) (width 0.381) (layer "B.Cu") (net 7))
 (segment (start 117.856 128.2192) (end 119.9388 130.302) (width 0.381) (layer "B.Cu") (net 18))
 (segment (start 119.9388 130.302) (end 119.9388 138.250589) (width 0.381) (layer "B.Cu") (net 18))
 (segment (start 119.94 138.251789) (end 119.94 139.4206) (width 0.381) (layer "B.Cu") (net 18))
 (segment (start 89.064945 128.2192) (end 117.856 128.2192) (width 0.381) (layer "B.Cu") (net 18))
 (segment (start 119.9388 138.250589) (end 119.94 138.251789) (width 0.381) (layer "B.Cu") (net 18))
 (segment (start 96.9796 126.2404) (end 96.9772 126.238) (width 0.381) (layer "B.Cu") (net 20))
 (segment (start 96.9796 126.2404) (end 90.6248 126.2404) (width 0.381) (layer "B.Cu") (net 20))
 (segment (start 125.02 128.322) (end 122.9384 126.2404) (width 0.381) (layer "B.Cu") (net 20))
 (segment (start 89.064945 126.2192) (end 90.6036 126.2192) (width 0.381) (layer "B.Cu") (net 20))
 (segment (start 125.02 139.4206) (end 125.02 128.322) (width 0.381) (layer "B.Cu") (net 20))
 (segment (start 90.2668 126.238) (end 90.229956 126.238) (width 0.381) (layer "B.Cu") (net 20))
 (segment (start 122.9384 126.2404) (end 96.9796 126.2404) (width 0.381) (layer "B.Cu") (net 20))
 (segment (start 90.2692 126.2404) (end 90.2668 126.238) (width 0.381) (layer "B.Cu") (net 20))
 (segment (start 90.6248 126.2404) (end 90.2692 126.2404) (width 0.381) (layer "B.Cu") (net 20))
 (segment (start 90.6036 126.2192) (end 90.6248 126.2404) (width 0.381) (layer "B.Cu") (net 20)))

